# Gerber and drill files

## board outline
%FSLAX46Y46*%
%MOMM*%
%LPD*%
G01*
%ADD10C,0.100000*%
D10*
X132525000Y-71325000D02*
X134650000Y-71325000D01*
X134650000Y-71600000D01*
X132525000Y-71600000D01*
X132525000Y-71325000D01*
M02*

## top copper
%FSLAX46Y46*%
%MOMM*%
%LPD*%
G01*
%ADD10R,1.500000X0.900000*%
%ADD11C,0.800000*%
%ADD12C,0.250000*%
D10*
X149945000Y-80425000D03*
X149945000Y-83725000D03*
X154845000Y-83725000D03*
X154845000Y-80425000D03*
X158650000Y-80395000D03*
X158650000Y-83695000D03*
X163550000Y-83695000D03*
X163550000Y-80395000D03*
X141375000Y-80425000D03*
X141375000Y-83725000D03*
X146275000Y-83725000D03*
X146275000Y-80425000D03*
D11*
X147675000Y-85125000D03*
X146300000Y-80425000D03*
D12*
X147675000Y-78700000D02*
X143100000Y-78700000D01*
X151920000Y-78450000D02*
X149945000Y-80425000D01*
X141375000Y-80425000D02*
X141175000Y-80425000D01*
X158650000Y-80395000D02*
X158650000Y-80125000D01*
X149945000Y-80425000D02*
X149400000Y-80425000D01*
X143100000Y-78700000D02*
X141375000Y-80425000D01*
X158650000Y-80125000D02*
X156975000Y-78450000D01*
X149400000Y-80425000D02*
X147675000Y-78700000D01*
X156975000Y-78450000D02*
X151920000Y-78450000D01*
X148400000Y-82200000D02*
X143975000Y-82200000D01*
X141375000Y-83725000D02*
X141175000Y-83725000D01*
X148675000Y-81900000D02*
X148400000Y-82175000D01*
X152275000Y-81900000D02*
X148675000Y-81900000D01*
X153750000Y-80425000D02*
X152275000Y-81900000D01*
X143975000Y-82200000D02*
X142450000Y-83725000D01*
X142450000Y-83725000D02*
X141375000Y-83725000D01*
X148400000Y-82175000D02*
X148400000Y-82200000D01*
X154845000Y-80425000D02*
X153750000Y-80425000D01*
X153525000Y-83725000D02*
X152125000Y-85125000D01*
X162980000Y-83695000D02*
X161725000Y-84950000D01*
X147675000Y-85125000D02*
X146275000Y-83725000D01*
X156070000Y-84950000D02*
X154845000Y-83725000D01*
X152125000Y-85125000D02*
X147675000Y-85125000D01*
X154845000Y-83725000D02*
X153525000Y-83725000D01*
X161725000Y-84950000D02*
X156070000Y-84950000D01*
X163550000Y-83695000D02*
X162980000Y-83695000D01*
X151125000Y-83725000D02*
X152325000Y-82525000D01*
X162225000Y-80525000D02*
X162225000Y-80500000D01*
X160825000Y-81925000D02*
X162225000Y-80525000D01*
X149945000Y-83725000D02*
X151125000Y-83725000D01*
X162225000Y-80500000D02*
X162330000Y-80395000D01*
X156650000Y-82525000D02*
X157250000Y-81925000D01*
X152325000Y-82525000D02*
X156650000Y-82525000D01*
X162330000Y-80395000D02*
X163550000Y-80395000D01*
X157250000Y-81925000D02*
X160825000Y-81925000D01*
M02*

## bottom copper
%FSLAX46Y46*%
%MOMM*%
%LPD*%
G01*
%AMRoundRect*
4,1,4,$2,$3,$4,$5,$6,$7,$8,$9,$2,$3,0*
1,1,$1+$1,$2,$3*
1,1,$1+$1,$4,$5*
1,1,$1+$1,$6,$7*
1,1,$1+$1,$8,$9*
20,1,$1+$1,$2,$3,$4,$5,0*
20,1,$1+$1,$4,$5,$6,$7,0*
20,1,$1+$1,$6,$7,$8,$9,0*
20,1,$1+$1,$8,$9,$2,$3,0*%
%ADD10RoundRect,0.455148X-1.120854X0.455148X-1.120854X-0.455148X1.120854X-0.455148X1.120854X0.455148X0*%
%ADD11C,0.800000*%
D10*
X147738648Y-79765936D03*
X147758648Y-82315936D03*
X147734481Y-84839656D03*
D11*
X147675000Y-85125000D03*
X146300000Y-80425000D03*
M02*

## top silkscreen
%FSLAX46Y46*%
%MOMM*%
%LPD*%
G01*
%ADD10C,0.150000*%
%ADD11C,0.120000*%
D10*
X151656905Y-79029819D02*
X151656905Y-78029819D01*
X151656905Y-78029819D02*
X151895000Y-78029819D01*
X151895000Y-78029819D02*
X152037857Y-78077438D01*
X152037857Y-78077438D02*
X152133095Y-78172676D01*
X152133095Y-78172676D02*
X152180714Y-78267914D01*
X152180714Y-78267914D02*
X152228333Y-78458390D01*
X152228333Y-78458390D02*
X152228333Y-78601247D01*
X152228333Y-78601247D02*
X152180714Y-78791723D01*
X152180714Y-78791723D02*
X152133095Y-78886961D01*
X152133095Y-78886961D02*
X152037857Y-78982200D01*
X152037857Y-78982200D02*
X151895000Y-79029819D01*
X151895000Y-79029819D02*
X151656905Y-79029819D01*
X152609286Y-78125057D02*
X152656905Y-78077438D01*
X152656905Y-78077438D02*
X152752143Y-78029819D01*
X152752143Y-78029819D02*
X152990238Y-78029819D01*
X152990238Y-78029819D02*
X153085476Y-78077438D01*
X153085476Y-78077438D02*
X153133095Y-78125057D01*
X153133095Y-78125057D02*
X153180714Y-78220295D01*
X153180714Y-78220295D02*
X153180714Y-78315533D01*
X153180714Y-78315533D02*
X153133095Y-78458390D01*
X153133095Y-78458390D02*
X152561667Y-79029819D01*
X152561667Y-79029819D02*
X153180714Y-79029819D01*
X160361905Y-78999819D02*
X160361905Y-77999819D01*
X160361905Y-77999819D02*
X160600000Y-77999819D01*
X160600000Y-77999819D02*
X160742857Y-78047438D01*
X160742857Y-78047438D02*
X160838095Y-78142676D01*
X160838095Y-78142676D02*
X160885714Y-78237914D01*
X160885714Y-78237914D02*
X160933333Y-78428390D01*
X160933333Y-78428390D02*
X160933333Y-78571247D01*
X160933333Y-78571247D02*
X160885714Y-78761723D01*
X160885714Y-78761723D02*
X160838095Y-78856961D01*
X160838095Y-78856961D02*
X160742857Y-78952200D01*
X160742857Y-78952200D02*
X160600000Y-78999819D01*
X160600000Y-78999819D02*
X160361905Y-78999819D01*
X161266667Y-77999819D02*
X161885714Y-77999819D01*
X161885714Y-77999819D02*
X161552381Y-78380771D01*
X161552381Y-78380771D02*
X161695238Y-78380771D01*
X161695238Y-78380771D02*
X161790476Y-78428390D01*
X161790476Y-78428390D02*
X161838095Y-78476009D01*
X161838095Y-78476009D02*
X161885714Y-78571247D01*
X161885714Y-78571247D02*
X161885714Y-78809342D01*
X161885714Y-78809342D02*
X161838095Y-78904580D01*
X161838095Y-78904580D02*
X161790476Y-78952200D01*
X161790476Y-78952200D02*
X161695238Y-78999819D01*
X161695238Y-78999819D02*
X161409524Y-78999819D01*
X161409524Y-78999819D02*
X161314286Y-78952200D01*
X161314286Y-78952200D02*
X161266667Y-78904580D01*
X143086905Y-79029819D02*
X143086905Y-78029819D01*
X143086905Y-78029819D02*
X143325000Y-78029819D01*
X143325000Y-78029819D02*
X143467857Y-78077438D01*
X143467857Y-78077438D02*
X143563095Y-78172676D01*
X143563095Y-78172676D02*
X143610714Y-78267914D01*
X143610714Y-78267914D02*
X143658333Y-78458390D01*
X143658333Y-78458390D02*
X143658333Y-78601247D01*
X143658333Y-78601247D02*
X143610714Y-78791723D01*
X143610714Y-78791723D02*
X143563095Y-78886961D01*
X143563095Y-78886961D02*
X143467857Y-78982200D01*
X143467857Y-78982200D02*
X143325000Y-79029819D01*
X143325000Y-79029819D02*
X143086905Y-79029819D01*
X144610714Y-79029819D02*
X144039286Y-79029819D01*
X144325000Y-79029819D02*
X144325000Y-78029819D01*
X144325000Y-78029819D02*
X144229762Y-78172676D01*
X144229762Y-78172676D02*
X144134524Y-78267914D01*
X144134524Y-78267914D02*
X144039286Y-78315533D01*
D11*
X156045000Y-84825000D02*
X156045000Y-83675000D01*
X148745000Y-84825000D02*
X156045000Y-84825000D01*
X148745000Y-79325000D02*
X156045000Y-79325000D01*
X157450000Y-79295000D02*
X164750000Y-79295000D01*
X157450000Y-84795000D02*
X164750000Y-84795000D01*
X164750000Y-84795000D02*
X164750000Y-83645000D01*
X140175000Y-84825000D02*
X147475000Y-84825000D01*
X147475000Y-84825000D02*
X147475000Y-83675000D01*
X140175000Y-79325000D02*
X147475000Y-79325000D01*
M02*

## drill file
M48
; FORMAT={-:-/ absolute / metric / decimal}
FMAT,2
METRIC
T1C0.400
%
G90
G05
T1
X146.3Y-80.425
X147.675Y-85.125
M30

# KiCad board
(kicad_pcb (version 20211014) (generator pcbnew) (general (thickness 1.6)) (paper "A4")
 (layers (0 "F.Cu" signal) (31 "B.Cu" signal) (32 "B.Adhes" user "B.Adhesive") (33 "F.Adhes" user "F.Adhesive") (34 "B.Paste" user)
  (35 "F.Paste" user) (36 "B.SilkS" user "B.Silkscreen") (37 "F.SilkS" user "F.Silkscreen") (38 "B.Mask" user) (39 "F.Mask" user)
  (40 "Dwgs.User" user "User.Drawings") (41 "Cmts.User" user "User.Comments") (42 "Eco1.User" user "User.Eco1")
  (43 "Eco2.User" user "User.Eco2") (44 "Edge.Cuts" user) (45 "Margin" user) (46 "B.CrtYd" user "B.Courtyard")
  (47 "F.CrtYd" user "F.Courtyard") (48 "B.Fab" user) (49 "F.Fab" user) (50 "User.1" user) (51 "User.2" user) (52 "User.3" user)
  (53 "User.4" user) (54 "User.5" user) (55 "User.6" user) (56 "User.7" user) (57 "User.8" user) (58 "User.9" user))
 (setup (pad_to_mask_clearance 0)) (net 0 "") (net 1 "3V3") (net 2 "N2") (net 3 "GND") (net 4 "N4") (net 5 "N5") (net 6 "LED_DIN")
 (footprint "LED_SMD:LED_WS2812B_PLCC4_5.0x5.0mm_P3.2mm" (layer "F.Cu") (at 152.395 82.075)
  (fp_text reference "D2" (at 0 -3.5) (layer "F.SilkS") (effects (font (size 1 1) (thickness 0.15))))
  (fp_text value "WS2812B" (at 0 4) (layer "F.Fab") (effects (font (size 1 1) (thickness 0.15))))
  (fp_line (start 3.65 2.75) (end 3.65 1.6) (layer "F.SilkS") (width 0.12))
  (fp_line (start -3.65 2.75) (end 3.65 2.75) (layer "F.SilkS") (width 0.12))
  (fp_line (start -3.65 -2.75) (end 3.65 -2.75) (layer "F.SilkS") (width 0.12))
  (pad "1" smd rect (at -2.45 -1.65) (size 1.5 0.9) (layers "F.Cu" "F.Paste" "F.Mask") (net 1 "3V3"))
  (pad "2" smd rect (at -2.45 1.65) (size 1.5 0.9) (layers "F.Cu" "F.Paste" "F.Mask") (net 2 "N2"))
  (pad "3" smd rect (at 2.45 1.65) (size 1.5 0.9) (layers "F.Cu" "F.Paste" "F.Mask") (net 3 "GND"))
  (pad "4" smd rect (at 2.45 -1.65) (size 1.5 0.9) (layers "F.Cu" "F.Paste" "F.Mask") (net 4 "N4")))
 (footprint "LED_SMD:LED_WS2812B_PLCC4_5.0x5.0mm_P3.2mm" (layer "F.Cu") (at 161.1 82.045)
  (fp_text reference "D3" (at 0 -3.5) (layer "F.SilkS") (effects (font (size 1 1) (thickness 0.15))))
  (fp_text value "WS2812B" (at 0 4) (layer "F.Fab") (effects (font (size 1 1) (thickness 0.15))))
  (fp_line (start -3.65 -2.75) (end 3.65 -2.75) (layer "F.SilkS") (width 0.12))
  (fp_line (start -3.65 2.75) (end 3.65 2.75) (layer "F.SilkS") (width 0.12))
  (fp_line (start 3.65 2.75) (end 3.65 1.6) (layer "F.SilkS") (width 0.12))
  (pad "1" smd rect (at -2.45 -1.65) (size 1.5 0.9) (layers "F.Cu" "F.Paste" "F.Mask") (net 1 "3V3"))
  (pad "2" smd rect (at -2.45 1.65) (size 1.5 0.9) (layers "F.Cu" "F.Paste" "F.Mask") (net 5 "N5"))
  (pad "3" smd rect (at 2.45 1.65) (size 1.5 0.9) (layers "F.Cu" "F.Paste" "F.Mask") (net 3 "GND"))
  (pad "4" smd rect (at 2.45 -1.65) (size 1.5 0.9) (layers "F.Cu" "F.Paste" "F.Mask") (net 2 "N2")))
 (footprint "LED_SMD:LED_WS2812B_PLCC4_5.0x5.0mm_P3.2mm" (layer "F.Cu") (at 143.825 82.075)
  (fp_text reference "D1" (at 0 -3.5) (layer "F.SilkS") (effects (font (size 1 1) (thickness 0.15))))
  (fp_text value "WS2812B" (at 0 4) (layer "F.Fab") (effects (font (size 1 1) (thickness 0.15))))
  (fp_line (start -3.65 2.75) (end 3.65 2.75) (layer "F.SilkS") (width 0.12))
  (fp_line (start 3.65 2.75) (end 3.65 1.6) (layer "F.SilkS") (width 0.12))
  (fp_line (start -3.65 -2.75) (end 3.65 -2.75) (layer "F.SilkS") (width 0.12))
  (pad "1" smd rect (at -2.45 -1.65) (size 1.5 0.9) (layers "F.Cu" "F.Paste" "F.Mask") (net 1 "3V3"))
  (pad "2" smd rect (at -2.45 1.65) (size 1.5 0.9) (layers "F.Cu" "F.Paste" "F.Mask") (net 4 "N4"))
  (pad "3" smd rect (at 2.45 1.65) (size 1.5 0.9) (layers "F.Cu" "F.Paste" "F.Mask") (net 3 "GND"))
  (pad "4" smd rect (at 2.45 -1.65) (size 1.5 0.9) (layers "F.Cu" "F.Paste" "F.Mask") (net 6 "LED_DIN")))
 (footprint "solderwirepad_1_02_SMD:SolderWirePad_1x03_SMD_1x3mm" (layer "B.Cu") (at 147.77 79.789167 -90)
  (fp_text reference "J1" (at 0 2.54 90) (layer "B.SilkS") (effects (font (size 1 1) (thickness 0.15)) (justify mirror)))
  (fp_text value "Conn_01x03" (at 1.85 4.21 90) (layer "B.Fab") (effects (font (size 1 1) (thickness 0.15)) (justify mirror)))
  (pad "1" smd roundrect (at -0.023231 0.031352 270) (size 1.820592 3.152005) (layers "B.Cu" "B.Paste" "B.Mask") (roundrect_rratio 0.25)
   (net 6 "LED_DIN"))
  (pad "2" smd roundrect (at 2.526769 0.011352 270) (size 1.820592 3.152005) (layers "B.Cu" "B.Paste" "B.Mask") (roundrect_rratio 0.25)
   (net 1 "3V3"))
  (pad "3" smd roundrect (at 5.050489 0.035519 270) (size 1.820592 3.152005) (layers "B.Cu" "B.Paste" "B.Mask") (roundrect_rratio 0.25)
   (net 3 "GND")))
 (gr_rect (start 132.525 71.6) (end 134.65 71.325) (layer "Edge.Cuts") (width 0.1) (fill none))
 (segment (start 147.675 78.7) (end 143.1 78.7) (width 0.25) (layer "F.Cu") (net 1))
 (segment (start 151.92 78.45) (end 149.945 80.425) (width 0.25) (layer "F.Cu") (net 1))
 (segment (start 141.375 80.425) (end 141.175 80.425) (width 0.25) (layer "F.Cu") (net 1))
 (segment (start 158.65 80.395) (end 158.65 80.125) (width 0.25) (layer "F.Cu") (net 1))
 (segment (start 149.945 80.425) (end 149.4 80.425) (width 0.25) (layer "F.Cu") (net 1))
 (segment (start 143.1 78.7) (end 141.375 80.425) (width 0.25) (layer "F.Cu") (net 1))
 (segment (start 158.65 80.125) (end 156.975 78.45) (width 0.25) (layer "F.Cu") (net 1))
 (segment (start 149.4 80.425) (end 147.675 78.7) (width 0.25) (layer "F.Cu") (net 1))
 (segment (start 156.975 78.45) (end 151.92 78.45) (width 0.25) (layer "F.Cu") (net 1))
 (segment (start 148.4 82.2) (end 143.975 82.2) (width 0.25) (layer "F.Cu") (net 4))
 (segment (start 141.375 83.725) (end 141.175 83.725) (width 0.25) (layer "F.Cu") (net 4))
 (segment (start 148.675 81.9) (end 148.4 82.175) (width 0.25) (layer "F.Cu") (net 4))
 (segment (start 152.275 81.9) (end 148.675 81.9) (width 0.25) (layer "F.Cu") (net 4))
 (segment (start 153.75 80.425) (end 152.275 81.9) (width 0.25) (layer "F.Cu") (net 4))
 (segment (start 143.975 82.2) (end 142.45 83.725) (width 0.25) (layer "F.Cu") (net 4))
 (segment (start 142.45 83.725) (end 141.375 83.725) (width 0.25) (layer "F.Cu") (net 4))
 (segment (start 148.4 82.175) (end 148.4 82.2) (width 0.25) (layer "F.Cu") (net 4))
 (segment (start 154.845 80.425) (end 153.75 80.425) (width 0.25) (layer "F.Cu") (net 4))
 (segment (start 153.525 83.725) (end 152.125 85.125) (width 0.25) (layer "F.Cu") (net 3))
 (segment (start 162.98 83.695) (end 161.725 84.95) (width 0.25) (layer "F.Cu") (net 3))
 (segment (start 147.675 85.125) (end 146.275 83.725) (width 0.25) (layer "F.Cu") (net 3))
 (segment (start 156.07 84.95) (end 154.845 83.725) (width 0.25) (layer "F.Cu") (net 3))
 (segment (start 152.125 85.125) (end 147.675 85.125) (width 0.25) (layer "F.Cu") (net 3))
 (segment (start 154.845 83.725) (end 153.525 83.725) (width 0.25) (layer "F.Cu") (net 3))
 (segment (start 161.725 84.95) (end 156.07 84.95) (width 0.25) (layer "F.Cu") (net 3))
 (segment (start 163.55 83.695) (end 162.98 83.695) (width 0.25) (layer "F.Cu") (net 3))
 (via (at 147.675 85.125) (size 0.8) (drill 0.4) (layers "F.Cu" "B.Cu") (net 3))
 (via (at 146.3 80.425) (size 0.8) (drill 0.4) (layers "F.Cu" "B.Cu") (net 6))
 (segment (start 151.125 83.725) (end 152.325 82.525) (width 0.25) (layer "F.Cu") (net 2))
 (segment (start 162.225 80.525) (end 162.225 80.5) (width 0.25) (layer "F.Cu") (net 2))
 (segment (start 160.825 81.925) (end 162.225 80.525) (width 0.25) (layer "F.Cu") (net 2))
 (segment (start 149.945 83.725) (end 151.125 83.725) (width 0.25) (layer "F.Cu") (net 2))
 (segment (start 162.225 80.5) (end 162.33 80.395) (width 0.25) (layer "F.Cu") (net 2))
 (segment (start 156.65 82.525) (end 157.25 81.925) (width 0.25) (layer "F.Cu") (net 2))
 (segment (start 152.325 82.525) (end 156.65 82.525) (width 0.25) (layer "F.Cu") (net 2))
 (segment (start 162.33 80.395) (end 163.55 80.395) (width 0.25) (layer "F.Cu") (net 2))
 (segment (start 157.25 81.925) (end 160.825 81.925) (width 0.25) (layer "F.Cu") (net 2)))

